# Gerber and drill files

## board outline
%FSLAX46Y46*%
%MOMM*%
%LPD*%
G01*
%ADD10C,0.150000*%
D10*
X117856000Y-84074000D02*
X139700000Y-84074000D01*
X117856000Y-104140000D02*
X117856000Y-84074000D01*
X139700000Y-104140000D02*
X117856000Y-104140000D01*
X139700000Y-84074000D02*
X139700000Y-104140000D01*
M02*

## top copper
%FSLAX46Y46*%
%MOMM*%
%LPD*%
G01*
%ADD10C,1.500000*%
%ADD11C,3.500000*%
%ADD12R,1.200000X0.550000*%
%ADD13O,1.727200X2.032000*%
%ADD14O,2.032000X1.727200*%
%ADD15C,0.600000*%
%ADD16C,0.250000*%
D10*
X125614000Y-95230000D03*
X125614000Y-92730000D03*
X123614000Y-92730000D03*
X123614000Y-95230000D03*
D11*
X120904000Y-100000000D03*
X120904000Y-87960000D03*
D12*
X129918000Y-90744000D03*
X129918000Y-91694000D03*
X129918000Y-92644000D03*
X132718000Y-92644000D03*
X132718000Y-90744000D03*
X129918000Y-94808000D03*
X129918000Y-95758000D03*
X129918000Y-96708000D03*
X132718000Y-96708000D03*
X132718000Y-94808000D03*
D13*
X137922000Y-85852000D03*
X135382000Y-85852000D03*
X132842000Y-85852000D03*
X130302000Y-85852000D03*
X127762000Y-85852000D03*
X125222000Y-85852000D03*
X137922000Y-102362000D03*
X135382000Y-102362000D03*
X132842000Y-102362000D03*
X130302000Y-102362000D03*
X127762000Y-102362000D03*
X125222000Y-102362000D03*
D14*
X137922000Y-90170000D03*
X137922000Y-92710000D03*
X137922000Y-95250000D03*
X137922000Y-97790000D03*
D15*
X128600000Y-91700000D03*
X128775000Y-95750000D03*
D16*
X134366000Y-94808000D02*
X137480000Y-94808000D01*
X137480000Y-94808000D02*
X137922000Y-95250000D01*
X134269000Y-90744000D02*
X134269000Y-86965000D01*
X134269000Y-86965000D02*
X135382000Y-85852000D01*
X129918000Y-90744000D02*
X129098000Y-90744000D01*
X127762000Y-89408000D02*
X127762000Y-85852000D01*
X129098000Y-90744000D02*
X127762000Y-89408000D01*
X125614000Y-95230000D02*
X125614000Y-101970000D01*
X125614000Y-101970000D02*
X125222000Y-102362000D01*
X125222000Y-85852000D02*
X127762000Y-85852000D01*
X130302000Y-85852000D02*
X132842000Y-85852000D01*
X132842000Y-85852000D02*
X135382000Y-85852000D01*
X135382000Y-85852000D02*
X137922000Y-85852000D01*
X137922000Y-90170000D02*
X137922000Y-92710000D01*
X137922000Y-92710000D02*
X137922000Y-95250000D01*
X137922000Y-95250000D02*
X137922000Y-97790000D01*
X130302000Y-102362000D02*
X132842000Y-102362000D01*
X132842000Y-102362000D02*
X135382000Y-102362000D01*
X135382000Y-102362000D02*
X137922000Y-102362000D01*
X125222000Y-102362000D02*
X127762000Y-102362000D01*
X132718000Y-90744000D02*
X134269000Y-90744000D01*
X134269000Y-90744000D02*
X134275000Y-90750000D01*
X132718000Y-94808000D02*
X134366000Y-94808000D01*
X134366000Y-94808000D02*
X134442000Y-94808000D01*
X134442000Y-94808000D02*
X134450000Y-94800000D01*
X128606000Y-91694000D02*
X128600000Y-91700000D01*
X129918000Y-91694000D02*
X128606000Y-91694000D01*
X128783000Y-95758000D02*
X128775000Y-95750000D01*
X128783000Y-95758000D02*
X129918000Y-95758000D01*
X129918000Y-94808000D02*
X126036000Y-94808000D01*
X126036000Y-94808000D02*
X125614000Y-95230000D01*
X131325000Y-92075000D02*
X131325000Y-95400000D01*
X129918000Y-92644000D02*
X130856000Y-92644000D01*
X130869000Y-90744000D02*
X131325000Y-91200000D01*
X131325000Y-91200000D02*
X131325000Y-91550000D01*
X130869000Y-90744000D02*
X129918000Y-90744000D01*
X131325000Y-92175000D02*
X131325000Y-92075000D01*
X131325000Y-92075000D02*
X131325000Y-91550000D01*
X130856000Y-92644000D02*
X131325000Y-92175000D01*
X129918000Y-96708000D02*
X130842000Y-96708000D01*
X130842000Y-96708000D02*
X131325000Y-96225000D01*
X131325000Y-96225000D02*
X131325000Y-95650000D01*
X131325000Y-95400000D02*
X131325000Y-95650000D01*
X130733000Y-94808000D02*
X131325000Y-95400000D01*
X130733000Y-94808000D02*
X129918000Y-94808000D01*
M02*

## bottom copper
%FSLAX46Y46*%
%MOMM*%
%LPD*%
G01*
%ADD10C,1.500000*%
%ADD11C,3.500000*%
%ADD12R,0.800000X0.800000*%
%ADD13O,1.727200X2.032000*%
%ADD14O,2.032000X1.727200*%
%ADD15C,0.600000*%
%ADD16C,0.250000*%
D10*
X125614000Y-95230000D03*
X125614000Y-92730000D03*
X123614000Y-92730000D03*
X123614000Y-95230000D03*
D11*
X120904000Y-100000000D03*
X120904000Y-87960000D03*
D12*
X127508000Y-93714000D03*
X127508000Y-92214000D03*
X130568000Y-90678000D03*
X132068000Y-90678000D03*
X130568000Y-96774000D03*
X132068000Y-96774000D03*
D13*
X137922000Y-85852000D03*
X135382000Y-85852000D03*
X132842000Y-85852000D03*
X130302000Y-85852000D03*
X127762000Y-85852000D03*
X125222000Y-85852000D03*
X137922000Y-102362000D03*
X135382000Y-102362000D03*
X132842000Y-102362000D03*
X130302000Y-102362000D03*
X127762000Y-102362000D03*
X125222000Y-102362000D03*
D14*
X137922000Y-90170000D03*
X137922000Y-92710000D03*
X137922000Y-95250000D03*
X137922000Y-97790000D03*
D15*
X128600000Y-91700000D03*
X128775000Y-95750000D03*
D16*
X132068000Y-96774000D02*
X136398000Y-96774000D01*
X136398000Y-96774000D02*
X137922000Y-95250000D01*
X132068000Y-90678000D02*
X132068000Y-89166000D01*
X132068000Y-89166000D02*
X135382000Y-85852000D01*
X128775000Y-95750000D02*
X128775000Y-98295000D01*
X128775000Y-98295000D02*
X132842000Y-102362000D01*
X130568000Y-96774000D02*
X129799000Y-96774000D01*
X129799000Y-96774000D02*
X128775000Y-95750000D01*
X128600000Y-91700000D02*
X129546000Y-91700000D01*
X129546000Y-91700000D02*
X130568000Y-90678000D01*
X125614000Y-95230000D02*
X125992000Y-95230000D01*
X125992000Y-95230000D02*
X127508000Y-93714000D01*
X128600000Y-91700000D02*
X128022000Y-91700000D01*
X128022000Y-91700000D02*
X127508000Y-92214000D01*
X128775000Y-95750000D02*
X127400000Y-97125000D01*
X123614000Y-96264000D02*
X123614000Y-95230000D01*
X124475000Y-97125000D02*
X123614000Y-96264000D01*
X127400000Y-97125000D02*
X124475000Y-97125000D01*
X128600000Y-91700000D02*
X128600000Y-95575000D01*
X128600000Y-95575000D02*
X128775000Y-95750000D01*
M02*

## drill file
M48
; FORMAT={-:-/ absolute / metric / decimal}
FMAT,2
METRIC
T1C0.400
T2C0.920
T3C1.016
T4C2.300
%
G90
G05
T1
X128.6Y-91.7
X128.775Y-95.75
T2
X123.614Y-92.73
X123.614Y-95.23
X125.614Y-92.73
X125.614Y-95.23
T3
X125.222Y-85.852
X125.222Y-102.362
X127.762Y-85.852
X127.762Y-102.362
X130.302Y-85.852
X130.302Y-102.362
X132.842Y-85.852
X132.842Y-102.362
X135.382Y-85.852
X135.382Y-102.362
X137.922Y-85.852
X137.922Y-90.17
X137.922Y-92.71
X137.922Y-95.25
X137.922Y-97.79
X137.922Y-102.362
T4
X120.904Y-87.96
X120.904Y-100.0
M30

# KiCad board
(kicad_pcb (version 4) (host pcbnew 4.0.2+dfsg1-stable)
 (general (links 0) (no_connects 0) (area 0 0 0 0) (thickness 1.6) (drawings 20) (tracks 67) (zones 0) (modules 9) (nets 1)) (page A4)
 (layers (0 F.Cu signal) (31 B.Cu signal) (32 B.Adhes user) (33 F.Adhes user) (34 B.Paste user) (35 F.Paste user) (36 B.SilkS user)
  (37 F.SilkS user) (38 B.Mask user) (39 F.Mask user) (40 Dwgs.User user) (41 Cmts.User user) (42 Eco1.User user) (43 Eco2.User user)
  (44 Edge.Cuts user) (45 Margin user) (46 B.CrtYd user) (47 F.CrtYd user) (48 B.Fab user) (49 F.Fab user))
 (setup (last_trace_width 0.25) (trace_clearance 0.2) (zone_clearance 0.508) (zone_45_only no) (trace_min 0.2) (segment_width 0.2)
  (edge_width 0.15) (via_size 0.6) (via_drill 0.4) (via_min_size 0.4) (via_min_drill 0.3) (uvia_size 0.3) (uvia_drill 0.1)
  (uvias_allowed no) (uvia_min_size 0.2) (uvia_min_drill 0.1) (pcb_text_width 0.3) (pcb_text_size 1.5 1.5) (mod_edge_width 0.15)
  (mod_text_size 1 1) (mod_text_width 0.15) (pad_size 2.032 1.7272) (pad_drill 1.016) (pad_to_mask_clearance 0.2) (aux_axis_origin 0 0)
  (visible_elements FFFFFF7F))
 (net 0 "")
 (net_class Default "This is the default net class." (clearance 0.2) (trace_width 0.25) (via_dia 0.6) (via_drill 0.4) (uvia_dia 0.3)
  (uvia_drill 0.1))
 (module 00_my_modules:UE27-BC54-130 (layer F.Cu) (at 120.904 93.98 270)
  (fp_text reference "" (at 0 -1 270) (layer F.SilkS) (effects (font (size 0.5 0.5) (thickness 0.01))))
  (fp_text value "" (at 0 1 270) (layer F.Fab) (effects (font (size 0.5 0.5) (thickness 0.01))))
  (pad V thru_hole circle (at 1.25 -4.71 270) (size 1.5 1.5) (drill 0.92) (layers *.Cu *.Mask F.SilkS))
  (pad - thru_hole circle (at -1.25 -4.71 270) (size 1.5 1.5) (drill 0.92) (layers *.Cu *.Mask F.SilkS))
  (pad + thru_hole circle (at -1.25 -2.71 270) (size 1.5 1.5) (drill 0.92) (layers *.Cu *.Mask F.SilkS))
  (pad G thru_hole circle (at 1.25 -2.71 270) (size 1.5 1.5) (drill 0.92) (layers *.Cu *.Mask F.SilkS))
  (pad X thru_hole circle (at 6.02 0 270) (size 3.5 3.5) (drill 2.3) (layers *.Cu *.Mask F.SilkS))
  (pad X thru_hole circle (at -6.02 0 270) (size 3.5 3.5) (drill 2.3) (layers *.Cu *.Mask F.SilkS)))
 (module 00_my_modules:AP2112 (layer F.Cu) (at 131.318 91.694)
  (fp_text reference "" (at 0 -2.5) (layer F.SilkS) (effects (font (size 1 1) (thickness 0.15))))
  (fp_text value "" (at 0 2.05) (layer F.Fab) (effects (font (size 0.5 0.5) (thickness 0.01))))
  (pad VIN smd rect (at -1.4 -0.95) (size 1.2 0.55) (layers F.Cu F.Paste F.Mask))
  (pad GND smd rect (at -1.4 0) (size 1.2 0.55) (layers F.Cu F.Paste F.Mask))
  (pad EN smd rect (at -1.4 0.95) (size 1.2 0.55) (layers F.Cu F.Paste F.Mask))
  (pad NC smd rect (at 1.4 0.95) (size 1.2 0.55) (layers F.Cu F.Paste F.Mask))
  (pad VOUT smd rect (at 1.4 -0.95) (size 1.2 0.55) (layers F.Cu F.Paste F.Mask)))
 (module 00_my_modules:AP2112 (layer F.Cu) (at 131.318 95.758)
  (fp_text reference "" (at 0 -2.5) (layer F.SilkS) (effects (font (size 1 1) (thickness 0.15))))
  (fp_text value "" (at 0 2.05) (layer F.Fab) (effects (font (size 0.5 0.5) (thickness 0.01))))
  (pad VIN smd rect (at -1.4 -0.95) (size 1.2 0.55) (layers F.Cu F.Paste F.Mask))
  (pad GND smd rect (at -1.4 0) (size 1.2 0.55) (layers F.Cu F.Paste F.Mask))
  (pad EN smd rect (at -1.4 0.95) (size 1.2 0.55) (layers F.Cu F.Paste F.Mask))
  (pad NC smd rect (at 1.4 0.95) (size 1.2 0.55) (layers F.Cu F.Paste F.Mask))
  (pad VOUT smd rect (at 1.4 -0.95) (size 1.2 0.55) (layers F.Cu F.Paste F.Mask)))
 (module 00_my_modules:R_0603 (layer B.Cu) (at 127.508 92.964 90)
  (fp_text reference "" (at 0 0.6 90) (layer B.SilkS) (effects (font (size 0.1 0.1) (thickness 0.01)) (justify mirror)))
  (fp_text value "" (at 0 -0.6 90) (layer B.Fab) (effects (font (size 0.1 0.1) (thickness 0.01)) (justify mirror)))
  (pad 1 smd rect (at -0.75 0 90) (size 0.8 0.8) (layers B.Cu B.Paste B.Mask))
  (pad 2 smd rect (at 0.75 0 90) (size 0.8 0.8) (layers B.Cu B.Paste B.Mask)))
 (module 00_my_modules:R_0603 (layer B.Cu) (at 131.318 90.678)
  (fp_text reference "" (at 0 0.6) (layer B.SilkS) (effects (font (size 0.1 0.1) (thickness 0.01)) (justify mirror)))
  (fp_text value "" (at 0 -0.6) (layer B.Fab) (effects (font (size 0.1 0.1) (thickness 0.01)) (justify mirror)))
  (pad 1 smd rect (at -0.75 0) (size 0.8 0.8) (layers B.Cu B.Paste B.Mask))
  (pad 2 smd rect (at 0.75 0) (size 0.8 0.8) (layers B.Cu B.Paste B.Mask)))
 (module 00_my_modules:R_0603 (layer B.Cu) (at 131.318 96.774)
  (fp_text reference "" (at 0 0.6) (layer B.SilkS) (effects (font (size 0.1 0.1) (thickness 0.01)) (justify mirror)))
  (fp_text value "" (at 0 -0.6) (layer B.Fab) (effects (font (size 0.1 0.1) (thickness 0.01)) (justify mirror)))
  (pad 1 smd rect (at -0.75 0) (size 0.8 0.8) (layers B.Cu B.Paste B.Mask))
  (pad 2 smd rect (at 0.75 0) (size 0.8 0.8) (layers B.Cu B.Paste B.Mask)))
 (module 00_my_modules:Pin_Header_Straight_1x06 (layer F.Cu) (at 137.922 85.852 270)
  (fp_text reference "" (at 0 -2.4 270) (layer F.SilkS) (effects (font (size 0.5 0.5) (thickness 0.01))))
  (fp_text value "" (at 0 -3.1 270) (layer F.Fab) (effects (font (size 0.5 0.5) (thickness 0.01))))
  (pad 1 thru_hole oval (at 0 0 270) (size 2.032 1.7272) (drill 1.016) (layers *.Cu *.Mask F.SilkS))
  (pad 2 thru_hole oval (at 0 2.54 270) (size 2.032 1.7272) (drill 1.016) (layers *.Cu *.Mask F.SilkS))
  (pad 3 thru_hole oval (at 0 5.08 270) (size 2.032 1.7272) (drill 1.016) (layers *.Cu *.Mask F.SilkS))
  (pad 4 thru_hole oval (at 0 7.62 270) (size 2.032 1.7272) (drill 1.016) (layers *.Cu *.Mask F.SilkS))
  (pad 5 thru_hole oval (at 0 10.16 270) (size 2.032 1.7272) (drill 1.016) (layers *.Cu *.Mask F.SilkS))
  (pad 6 thru_hole oval (at 0 12.7 270) (size 2.032 1.7272) (drill 1.016) (layers *.Cu *.Mask F.SilkS)))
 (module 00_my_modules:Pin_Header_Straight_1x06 (layer F.Cu) (at 137.922 102.362 270)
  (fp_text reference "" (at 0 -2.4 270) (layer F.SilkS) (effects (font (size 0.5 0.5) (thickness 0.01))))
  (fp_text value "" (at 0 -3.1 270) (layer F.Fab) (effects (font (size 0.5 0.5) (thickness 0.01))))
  (pad 1 thru_hole oval (at 0 0 270) (size 2.032 1.7272) (drill 1.016) (layers *.Cu *.Mask F.SilkS))
  (pad 2 thru_hole oval (at 0 2.54 270) (size 2.032 1.7272) (drill 1.016) (layers *.Cu *.Mask F.SilkS))
  (pad 3 thru_hole oval (at 0 5.08 270) (size 2.032 1.7272) (drill 1.016) (layers *.Cu *.Mask F.SilkS))
  (pad 4 thru_hole oval (at 0 7.62 270) (size 2.032 1.7272) (drill 1.016) (layers *.Cu *.Mask F.SilkS))
  (pad 5 thru_hole oval (at 0 10.16 270) (size 2.032 1.7272) (drill 1.016) (layers *.Cu *.Mask F.SilkS))
  (pad 6 thru_hole oval (at 0 12.7 270) (size 2.032 1.7272) (drill 1.016) (layers *.Cu *.Mask F.SilkS)))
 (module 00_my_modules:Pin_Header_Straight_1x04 (layer F.Cu) (at 137.922 90.17)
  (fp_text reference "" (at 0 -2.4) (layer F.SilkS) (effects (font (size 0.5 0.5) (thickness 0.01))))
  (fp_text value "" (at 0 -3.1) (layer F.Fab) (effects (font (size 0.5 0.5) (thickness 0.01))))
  (pad 1 thru_hole oval (at 0 0) (size 2.032 1.7272) (drill 1.016) (layers *.Cu *.Mask F.SilkS))
  (pad 2 thru_hole oval (at 0 2.54) (size 2.032 1.7272) (drill 1.016) (layers *.Cu *.Mask F.SilkS))
  (pad 3 thru_hole oval (at 0 5.08) (size 2.032 1.7272) (drill 1.016) (layers *.Cu *.Mask F.SilkS))
  (pad 4 thru_hole oval (at 0 7.62) (size 2.032 1.7272) (drill 1.016) (layers *.Cu *.Mask F.SilkS)))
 (gr_line (start 117.856 84.074) (end 139.7 84.074) (angle 90) (layer Edge.Cuts) (width 0.15))
 (gr_line (start 117.856 104.14) (end 117.856 84.074) (angle 90) (layer Edge.Cuts) (width 0.15))
 (gr_line (start 139.7 104.14) (end 117.856 104.14) (angle 90) (layer Edge.Cuts) (width 0.15))
 (gr_line (start 139.7 84.074) (end 139.7 104.14) (angle 90) (layer Edge.Cuts) (width 0.15))
 (segment (start 134.366 94.808) (end 137.48 94.808) (width 0.25) (layer F.Cu) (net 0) (status 800000))
 (segment (start 137.48 94.808) (end 137.922 95.25) (width 0.25) (layer F.Cu) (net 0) (status C00000))
 (segment (start 132.068 96.774) (end 136.398 96.774) (width 0.25) (layer B.Cu) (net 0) (status 400000))
 (segment (start 136.398 96.774) (end 137.922 95.25) (width 0.25) (layer B.Cu) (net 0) (status 800000))
 (segment (start 132.068 90.678) (end 132.068 89.166) (width 0.25) (layer B.Cu) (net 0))
 (segment (start 132.068 89.166) (end 135.382 85.852) (width 0.25) (layer B.Cu) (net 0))
 (segment (start 128.775 95.75) (end 128.775 98.295) (width 0.25) (layer B.Cu) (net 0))
 (segment (start 128.775 98.295) (end 132.842 102.362) (width 0.25) (layer B.Cu) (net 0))
 (segment (start 134.269 90.744) (end 134.269 86.965) (width 0.25) (layer F.Cu) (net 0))
 (segment (start 134.269 86.965) (end 135.382 85.852) (width 0.25) (layer F.Cu) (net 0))
 (segment (start 129.918 90.744) (end 129.098 90.744) (width 0.25) (layer F.Cu) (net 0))
 (segment (start 127.762 89.408) (end 127.762 85.852) (width 0.25) (layer F.Cu) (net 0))
 (segment (start 129.098 90.744) (end 127.762 89.408) (width 0.25) (layer F.Cu) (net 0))
 (segment (start 125.614 95.23) (end 125.614 101.97) (width 0.25) (layer F.Cu) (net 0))
 (segment (start 125.614 101.97) (end 125.222 102.362) (width 0.25) (layer F.Cu) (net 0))
 (segment (start 125.222 85.852) (end 127.762 85.852) (width 0.25) (layer F.Cu) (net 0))
 (segment (start 130.302 85.852) (end 132.842 85.852) (width 0.25) (layer F.Cu) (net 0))
 (segment (start 132.842 85.852) (end 135.382 85.852) (width 0.25) (layer F.Cu) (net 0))
 (segment (start 135.382 85.852) (end 137.922 85.852) (width 0.25) (layer F.Cu) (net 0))
 (segment (start 137.922 90.17) (end 137.922 92.71) (width 0.25) (layer F.Cu) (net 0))
 (segment (start 137.922 92.71) (end 137.922 95.25) (width 0.25) (layer F.Cu) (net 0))
 (segment (start 137.922 95.25) (end 137.922 97.79) (width 0.25) (layer F.Cu) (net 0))
 (segment (start 130.302 102.362) (end 132.842 102.362) (width 0.25) (layer F.Cu) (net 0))
 (segment (start 132.842 102.362) (end 135.382 102.362) (width 0.25) (layer F.Cu) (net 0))
 (segment (start 135.382 102.362) (end 137.922 102.362) (width 0.25) (layer F.Cu) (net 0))
 (segment (start 125.222 102.362) (end 127.762 102.362) (width 0.25) (layer F.Cu) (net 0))
 (segment (start 130.568 96.774) (end 129.799 96.774) (width 0.25) (layer B.Cu) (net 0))
 (segment (start 129.799 96.774) (end 128.775 95.75) (width 0.25) (layer B.Cu) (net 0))
 (segment (start 128.6 91.7) (end 129.546 91.7) (width 0.25) (layer B.Cu) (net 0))
 (segment (start 129.546 91.7) (end 130.568 90.678) (width 0.25) (layer B.Cu) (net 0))
 (segment (start 125.614 95.23) (end 125.992 95.23) (width 0.25) (layer B.Cu) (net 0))
 (segment (start 125.992 95.23) (end 127.508 93.714) (width 0.25) (layer B.Cu) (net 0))
 (segment (start 128.6 91.7) (end 128.022 91.7) (width 0.25) (layer B.Cu) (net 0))
 (segment (start 128.022 91.7) (end 127.508 92.214) (width 0.25) (layer B.Cu) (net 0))
 (segment (start 132.718 90.744) (end 134.269 90.744) (width 0.25) (layer F.Cu) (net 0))
 (segment (start 134.269 90.744) (end 134.275 90.75) (width 0.25) (layer F.Cu) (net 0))
 (segment (start 132.718 94.808) (end 134.366 94.808) (width 0.25) (layer F.Cu) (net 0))
 (segment (start 134.366 94.808) (end 134.442 94.808) (width 0.25) (layer F.Cu) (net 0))
 (segment (start 134.442 94.808) (end 134.45 94.8) (width 0.25) (layer F.Cu) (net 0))
 (segment (start 128.775 95.75) (end 127.4 97.125) (width 0.25) (layer B.Cu) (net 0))
 (segment (start 123.614 96.264) (end 123.614 95.23) (width 0.25) (layer B.Cu) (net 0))
 (segment (start 124.475 97.125) (end 123.614 96.264) (width 0.25) (layer B.Cu) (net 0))
 (segment (start 127.4 97.125) (end 124.475 97.125) (width 0.25) (layer B.Cu) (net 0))
 (segment (start 128.6 91.7) (end 128.6 95.575) (width 0.25) (layer B.Cu) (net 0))
 (segment (start 128.606 91.694) (end 128.6 91.7) (width 0.25) (layer F.Cu) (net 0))
 (via (at 128.6 91.7) (size 0.6) (drill 0.4) (layers F.Cu B.Cu) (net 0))
 (segment (start 129.918 91.694) (end 128.606 91.694) (width 0.25) (layer F.Cu) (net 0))
 (segment (start 128.783 95.758) (end 128.775 95.75) (width 0.25) (layer F.Cu) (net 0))
 (via (at 128.775 95.75) (size 0.6) (drill 0.4) (layers F.Cu B.Cu) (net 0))
 (segment (start 128.783 95.758) (end 129.918 95.758) (width 0.25) (layer F.Cu) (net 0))
 (segment (start 128.6 95.575) (end 128.775 95.75) (width 0.25) (layer B.Cu) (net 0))
 (segment (start 129.918 94.808) (end 126.036 94.808) (width 0.25) (layer F.Cu) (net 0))
 (segment (start 126.036 94.808) (end 125.614 95.23) (width 0.25) (layer F.Cu) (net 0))
 (segment (start 131.325 92.075) (end 131.325 95.4) (width 0.25) (layer F.Cu) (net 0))
 (segment (start 129.918 92.644) (end 130.856 92.644) (width 0.25) (layer F.Cu) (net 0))
 (segment (start 130.869 90.744) (end 131.325 91.2) (width 0.25) (layer F.Cu) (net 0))
 (segment (start 131.325 91.2) (end 131.325 91.55) (width 0.25) (layer F.Cu) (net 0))
 (segment (start 130.869 90.744) (end 129.918 90.744) (width 0.25) (layer F.Cu) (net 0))
 (segment (start 131.325 92.175) (end 131.325 92.075) (width 0.25) (layer F.Cu) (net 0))
 (segment (start 131.325 92.075) (end 131.325 91.55) (width 0.25) (layer F.Cu) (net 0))
 (segment (start 130.856 92.644) (end 131.325 92.175) (width 0.25) (layer F.Cu) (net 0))
 (segment (start 129.918 96.708) (end 130.842 96.708) (width 0.25) (layer F.Cu) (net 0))
 (segment (start 130.842 96.708) (end 131.325 96.225) (width 0.25) (layer F.Cu) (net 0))
 (segment (start 131.325 96.225) (end 131.325 95.65) (width 0.25) (layer F.Cu) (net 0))
 (segment (start 131.325 95.4) (end 131.325 95.65) (width 0.25) (layer F.Cu) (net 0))
 (segment (start 130.733 94.808) (end 131.325 95.4) (width 0.25) (layer F.Cu) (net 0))
 (segment (start 130.733 94.808) (end 129.918 94.808) (width 0.25) (layer F.Cu) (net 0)))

